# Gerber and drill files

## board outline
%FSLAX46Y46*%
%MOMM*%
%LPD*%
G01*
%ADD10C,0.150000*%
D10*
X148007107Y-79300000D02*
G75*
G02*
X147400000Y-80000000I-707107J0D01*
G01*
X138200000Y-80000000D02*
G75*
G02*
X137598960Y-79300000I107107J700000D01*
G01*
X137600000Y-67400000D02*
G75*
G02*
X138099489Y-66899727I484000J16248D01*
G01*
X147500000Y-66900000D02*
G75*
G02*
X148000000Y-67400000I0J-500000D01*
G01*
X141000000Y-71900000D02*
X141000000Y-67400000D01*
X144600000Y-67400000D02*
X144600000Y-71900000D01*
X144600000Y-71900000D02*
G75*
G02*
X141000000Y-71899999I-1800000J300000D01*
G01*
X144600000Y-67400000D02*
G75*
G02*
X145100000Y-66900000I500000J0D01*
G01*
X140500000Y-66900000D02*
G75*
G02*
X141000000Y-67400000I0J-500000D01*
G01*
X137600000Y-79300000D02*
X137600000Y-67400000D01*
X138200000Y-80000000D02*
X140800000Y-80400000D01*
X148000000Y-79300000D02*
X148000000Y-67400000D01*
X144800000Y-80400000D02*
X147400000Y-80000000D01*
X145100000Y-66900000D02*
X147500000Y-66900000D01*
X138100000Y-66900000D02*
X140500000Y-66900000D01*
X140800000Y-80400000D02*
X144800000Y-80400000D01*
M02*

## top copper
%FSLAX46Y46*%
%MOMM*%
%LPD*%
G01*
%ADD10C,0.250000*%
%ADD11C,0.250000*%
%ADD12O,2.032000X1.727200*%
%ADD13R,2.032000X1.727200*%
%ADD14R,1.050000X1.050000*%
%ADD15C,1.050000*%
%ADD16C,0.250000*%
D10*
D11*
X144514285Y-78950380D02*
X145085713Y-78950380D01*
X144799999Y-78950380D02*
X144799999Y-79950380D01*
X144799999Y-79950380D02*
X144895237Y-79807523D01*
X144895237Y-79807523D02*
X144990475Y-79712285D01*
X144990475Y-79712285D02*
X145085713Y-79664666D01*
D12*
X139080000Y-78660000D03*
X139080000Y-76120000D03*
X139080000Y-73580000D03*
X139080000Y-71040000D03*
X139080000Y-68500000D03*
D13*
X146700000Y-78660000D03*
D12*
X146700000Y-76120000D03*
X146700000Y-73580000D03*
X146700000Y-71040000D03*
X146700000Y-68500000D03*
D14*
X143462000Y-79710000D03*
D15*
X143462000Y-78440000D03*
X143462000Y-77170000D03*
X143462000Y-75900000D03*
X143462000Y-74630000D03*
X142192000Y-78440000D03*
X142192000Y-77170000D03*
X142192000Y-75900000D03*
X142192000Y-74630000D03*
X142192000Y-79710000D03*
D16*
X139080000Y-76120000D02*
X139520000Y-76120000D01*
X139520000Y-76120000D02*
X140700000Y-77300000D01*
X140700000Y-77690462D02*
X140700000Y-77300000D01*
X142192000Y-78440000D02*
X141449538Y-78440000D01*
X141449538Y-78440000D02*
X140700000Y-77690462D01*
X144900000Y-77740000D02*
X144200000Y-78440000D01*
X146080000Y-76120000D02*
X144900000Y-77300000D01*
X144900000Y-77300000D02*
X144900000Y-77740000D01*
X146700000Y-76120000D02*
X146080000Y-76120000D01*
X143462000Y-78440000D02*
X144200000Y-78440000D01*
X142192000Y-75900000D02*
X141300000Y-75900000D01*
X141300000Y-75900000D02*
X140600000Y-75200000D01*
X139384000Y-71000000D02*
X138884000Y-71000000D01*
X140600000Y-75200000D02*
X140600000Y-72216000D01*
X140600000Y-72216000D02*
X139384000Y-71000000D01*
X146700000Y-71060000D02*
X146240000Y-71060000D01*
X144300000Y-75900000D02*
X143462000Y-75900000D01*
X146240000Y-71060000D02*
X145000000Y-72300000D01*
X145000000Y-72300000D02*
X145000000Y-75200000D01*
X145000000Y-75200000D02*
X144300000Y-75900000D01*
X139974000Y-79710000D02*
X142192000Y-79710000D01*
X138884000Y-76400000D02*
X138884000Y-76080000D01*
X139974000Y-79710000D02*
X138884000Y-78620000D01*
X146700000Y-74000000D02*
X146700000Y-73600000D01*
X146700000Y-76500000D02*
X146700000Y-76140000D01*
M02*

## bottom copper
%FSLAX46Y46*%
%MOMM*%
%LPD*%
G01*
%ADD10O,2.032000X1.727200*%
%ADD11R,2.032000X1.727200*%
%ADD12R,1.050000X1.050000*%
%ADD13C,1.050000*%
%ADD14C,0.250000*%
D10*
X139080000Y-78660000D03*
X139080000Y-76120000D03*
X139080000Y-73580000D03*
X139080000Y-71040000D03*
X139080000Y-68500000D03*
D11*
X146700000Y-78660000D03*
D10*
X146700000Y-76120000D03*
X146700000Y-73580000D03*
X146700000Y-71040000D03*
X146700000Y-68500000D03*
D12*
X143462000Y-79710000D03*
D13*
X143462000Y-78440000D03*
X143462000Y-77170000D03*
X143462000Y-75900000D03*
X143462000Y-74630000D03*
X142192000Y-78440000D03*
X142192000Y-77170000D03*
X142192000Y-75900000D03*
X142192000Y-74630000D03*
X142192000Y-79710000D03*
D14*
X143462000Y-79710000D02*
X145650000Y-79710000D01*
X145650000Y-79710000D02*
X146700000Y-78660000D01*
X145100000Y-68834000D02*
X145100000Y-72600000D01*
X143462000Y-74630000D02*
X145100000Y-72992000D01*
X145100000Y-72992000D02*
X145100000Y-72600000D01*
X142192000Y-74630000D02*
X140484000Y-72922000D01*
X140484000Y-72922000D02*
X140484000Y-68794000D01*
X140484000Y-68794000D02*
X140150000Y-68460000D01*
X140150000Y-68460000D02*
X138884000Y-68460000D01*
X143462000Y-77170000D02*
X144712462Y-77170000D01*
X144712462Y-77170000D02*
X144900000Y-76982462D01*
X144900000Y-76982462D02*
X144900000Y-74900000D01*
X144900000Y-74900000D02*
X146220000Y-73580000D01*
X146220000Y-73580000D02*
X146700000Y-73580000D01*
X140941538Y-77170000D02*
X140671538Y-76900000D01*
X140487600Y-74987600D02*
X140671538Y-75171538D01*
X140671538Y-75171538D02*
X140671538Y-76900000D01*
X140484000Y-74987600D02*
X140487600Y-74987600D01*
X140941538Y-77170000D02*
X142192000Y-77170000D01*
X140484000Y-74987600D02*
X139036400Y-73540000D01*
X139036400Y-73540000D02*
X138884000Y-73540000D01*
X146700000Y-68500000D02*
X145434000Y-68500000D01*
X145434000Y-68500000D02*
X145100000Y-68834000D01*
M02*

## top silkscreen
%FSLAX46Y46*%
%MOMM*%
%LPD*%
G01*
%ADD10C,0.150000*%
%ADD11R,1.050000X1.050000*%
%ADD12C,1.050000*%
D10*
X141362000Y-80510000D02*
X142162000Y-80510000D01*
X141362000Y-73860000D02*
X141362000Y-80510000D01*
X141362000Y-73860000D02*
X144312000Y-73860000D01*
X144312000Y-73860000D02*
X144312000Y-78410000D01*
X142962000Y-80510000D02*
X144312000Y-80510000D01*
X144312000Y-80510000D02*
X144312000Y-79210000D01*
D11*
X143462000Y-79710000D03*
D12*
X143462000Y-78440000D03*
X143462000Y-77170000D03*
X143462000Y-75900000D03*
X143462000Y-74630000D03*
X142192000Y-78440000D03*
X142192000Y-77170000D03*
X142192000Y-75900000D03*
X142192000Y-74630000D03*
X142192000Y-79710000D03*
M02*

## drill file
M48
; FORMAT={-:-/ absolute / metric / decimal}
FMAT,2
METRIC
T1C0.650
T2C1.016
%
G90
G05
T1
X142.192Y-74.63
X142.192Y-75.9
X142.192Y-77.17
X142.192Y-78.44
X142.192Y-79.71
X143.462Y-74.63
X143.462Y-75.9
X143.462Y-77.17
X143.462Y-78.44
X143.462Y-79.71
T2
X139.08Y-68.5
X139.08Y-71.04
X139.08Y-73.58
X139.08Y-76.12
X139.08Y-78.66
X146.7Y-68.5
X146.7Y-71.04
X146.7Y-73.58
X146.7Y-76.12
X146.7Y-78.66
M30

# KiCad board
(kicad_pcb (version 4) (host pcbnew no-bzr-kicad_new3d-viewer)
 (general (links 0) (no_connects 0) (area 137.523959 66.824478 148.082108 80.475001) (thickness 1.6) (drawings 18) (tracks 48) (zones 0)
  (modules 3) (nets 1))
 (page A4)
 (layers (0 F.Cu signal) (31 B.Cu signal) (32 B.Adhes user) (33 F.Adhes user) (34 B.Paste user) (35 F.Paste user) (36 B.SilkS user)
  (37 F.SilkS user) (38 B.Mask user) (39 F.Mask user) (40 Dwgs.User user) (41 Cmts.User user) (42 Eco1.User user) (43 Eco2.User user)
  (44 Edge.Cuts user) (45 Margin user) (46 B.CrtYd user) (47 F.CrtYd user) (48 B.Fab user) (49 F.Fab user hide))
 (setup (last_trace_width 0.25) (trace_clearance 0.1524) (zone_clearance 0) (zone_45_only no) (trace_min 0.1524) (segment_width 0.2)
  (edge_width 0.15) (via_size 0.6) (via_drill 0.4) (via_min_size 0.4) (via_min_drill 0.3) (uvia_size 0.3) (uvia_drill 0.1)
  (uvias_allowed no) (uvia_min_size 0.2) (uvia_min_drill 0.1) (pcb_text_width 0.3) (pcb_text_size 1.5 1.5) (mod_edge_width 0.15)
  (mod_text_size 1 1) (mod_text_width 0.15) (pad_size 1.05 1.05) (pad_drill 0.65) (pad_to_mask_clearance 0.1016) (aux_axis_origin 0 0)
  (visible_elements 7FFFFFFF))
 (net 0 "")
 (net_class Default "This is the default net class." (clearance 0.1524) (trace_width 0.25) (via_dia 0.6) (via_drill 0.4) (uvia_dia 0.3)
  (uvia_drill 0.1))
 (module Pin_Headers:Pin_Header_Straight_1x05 (layer B.Cu) (at 139.08 78.66)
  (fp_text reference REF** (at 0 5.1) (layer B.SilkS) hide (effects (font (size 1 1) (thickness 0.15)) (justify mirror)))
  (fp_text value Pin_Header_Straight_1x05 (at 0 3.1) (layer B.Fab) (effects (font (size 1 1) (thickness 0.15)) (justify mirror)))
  (pad 1 thru_hole oval (at 0 0) (size 2.032 1.7272) (drill 1.016) (layers *.Cu *.Mask B.SilkS))
  (pad 2 thru_hole oval (at 0 -2.54) (size 2.032 1.7272) (drill 1.016) (layers *.Cu *.Mask B.SilkS))
  (pad 3 thru_hole oval (at 0 -5.08) (size 2.032 1.7272) (drill 1.016) (layers *.Cu *.Mask B.SilkS))
  (pad 4 thru_hole oval (at 0 -7.62) (size 2.032 1.7272) (drill 1.016) (layers *.Cu *.Mask B.SilkS))
  (pad 5 thru_hole oval (at 0 -10.16) (size 2.032 1.7272) (drill 1.016) (layers *.Cu *.Mask B.SilkS)))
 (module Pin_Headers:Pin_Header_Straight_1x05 (layer B.Cu) (at 146.7 78.66)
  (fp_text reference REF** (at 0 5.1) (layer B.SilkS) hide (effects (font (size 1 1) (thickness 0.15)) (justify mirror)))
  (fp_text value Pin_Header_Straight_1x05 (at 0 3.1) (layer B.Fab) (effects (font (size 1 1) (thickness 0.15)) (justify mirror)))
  (pad 1 thru_hole rect (at 0 0) (size 2.032 1.7272) (drill 1.016) (layers *.Cu *.Mask B.SilkS))
  (pad 2 thru_hole oval (at 0 -2.54) (size 2.032 1.7272) (drill 1.016) (layers *.Cu *.Mask B.SilkS))
  (pad 3 thru_hole oval (at 0 -5.08) (size 2.032 1.7272) (drill 1.016) (layers *.Cu *.Mask B.SilkS))
  (pad 4 thru_hole oval (at 0 -7.62) (size 2.032 1.7272) (drill 1.016) (layers *.Cu *.Mask B.SilkS))
  (pad 5 thru_hole oval (at 0 -10.16) (size 2.032 1.7272) (drill 1.016) (layers *.Cu *.Mask B.SilkS)))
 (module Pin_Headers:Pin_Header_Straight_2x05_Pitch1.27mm (layer F.Cu) (at 143.462 79.71 180)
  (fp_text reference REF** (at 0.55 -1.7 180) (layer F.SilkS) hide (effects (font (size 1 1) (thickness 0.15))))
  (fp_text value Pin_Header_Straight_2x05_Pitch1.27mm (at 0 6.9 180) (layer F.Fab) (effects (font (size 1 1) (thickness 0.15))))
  (fp_line (start 2.1 -0.8) (end 1.3 -0.8) (layer F.SilkS) (width 0.15))
  (fp_line (start 2.1 5.85) (end 2.1 -0.8) (layer F.SilkS) (width 0.15))
  (fp_line (start 2.1 5.85) (end -0.85 5.85) (layer F.SilkS) (width 0.15))
  (fp_line (start -0.85 5.85) (end -0.85 1.3) (layer F.SilkS) (width 0.15))
  (fp_line (start 0.5 -0.8) (end -0.85 -0.8) (layer F.SilkS) (width 0.15))
  (fp_line (start -0.85 -0.8) (end -0.85 0.5) (layer F.SilkS) (width 0.15))
  (pad 1 thru_hole rect (at 0 0 180) (size 1.05 1.05) (drill 0.65) (layers *.Cu *.Mask F.SilkS))
  (pad 3 thru_hole circle (at 0 1.27 180) (size 1.05 1.05) (drill 0.65) (layers *.Cu *.Mask F.SilkS))
  (pad 5 thru_hole circle (at 0 2.54 180) (size 1.05 1.05) (drill 0.65) (layers *.Cu *.Mask F.SilkS))
  (pad 7 thru_hole circle (at 0 3.81 180) (size 1.05 1.05) (drill 0.65) (layers *.Cu *.Mask F.SilkS))
  (pad 9 thru_hole circle (at 0 5.08 180) (size 1.05 1.05) (drill 0.65) (layers *.Cu *.Mask F.SilkS))
  (pad 4 thru_hole circle (at 1.27 1.27 180) (size 1.05 1.05) (drill 0.65) (layers *.Cu *.Mask F.SilkS))
  (pad 6 thru_hole circle (at 1.27 2.54 180) (size 1.05 1.05) (drill 0.65) (layers *.Cu *.Mask F.SilkS))
  (pad 8 thru_hole circle (at 1.27 3.81 180) (size 1.05 1.05) (drill 0.65) (layers *.Cu *.Mask F.SilkS))
  (pad 10 thru_hole circle (at 1.27 5.08 180) (size 1.05 1.05) (drill 0.65) (layers *.Cu *.Mask F.SilkS))
  (pad 2 thru_hole circle (at 1.27 0 180) (size 1.05 1.05) (drill 0.65) (layers *.Cu *.Mask F.SilkS)))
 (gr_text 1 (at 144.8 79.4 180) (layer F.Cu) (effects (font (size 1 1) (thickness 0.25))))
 (gr_arc (start 147.3 79.3) (end 147.4 80) (angle -81.86989765) (layer Edge.Cuts) (width 0.15))
 (gr_arc (start 138.307107 79.3) (end 138.2 80) (angle 81.30064399) (layer Edge.Cuts) (width 0.15))
 (gr_arc (start 138.084 67.383752) (end 137.6 67.4) (angle 93.75557462) (layer Edge.Cuts) (width 0.15))
 (gr_arc (start 147.5 67.4) (end 147.5 66.9) (angle 90) (layer Edge.Cuts) (width 0.15))
 (gr_line (start 141 71.9) (end 141 67.4) (layer Edge.Cuts) (width 0.15))
 (gr_line (start 144.6 67.4) (end 144.6 71.9) (layer Edge.Cuts) (width 0.15))
 (gr_arc (start 142.8 71.6) (end 144.6 71.9) (angle 161.0753866) (layer Edge.Cuts) (width 0.15))
 (gr_arc (start 145.1 67.4) (end 144.6 67.4) (angle 90) (layer Edge.Cuts) (width 0.15))
 (gr_arc (start 140.5 67.4) (end 140.5 66.9) (angle 90) (layer Edge.Cuts) (width 0.15))
 (gr_line (start 137.6 79.3) (end 137.6 67.4) (layer Edge.Cuts) (width 0.15))
 (gr_line (start 138.2 80) (end 140.8 80.4) (layer Edge.Cuts) (width 0.15))
 (gr_line (start 148 79.3) (end 148 67.4) (layer Edge.Cuts) (width 0.15))
 (gr_line (start 144.8 80.4) (end 147.4 80) (layer Edge.Cuts) (width 0.15))
 (gr_line (start 145.1 66.9) (end 147.5 66.9) (layer Edge.Cuts) (width 0.15))
 (gr_line (start 138.1 66.9) (end 140.5 66.9) (layer Edge.Cuts) (width 0.15))
 (gr_line (start 140.8 80.4) (end 144.8 80.4) (layer Edge.Cuts) (width 0.15))
 (segment (start 143.462 79.71) (end 145.65 79.71) (width 0.25) (layer B.Cu) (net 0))
 (segment (start 145.65 79.71) (end 146.7 78.66) (width 0.25) (layer B.Cu) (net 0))
 (segment (start 139.08 76.12) (end 139.52 76.12) (width 0.25) (layer F.Cu) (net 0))
 (segment (start 139.52 76.12) (end 140.7 77.3) (width 0.25) (layer F.Cu) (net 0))
 (segment (start 140.7 77.690462) (end 140.7 77.3) (width 0.25) (layer F.Cu) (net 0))
 (segment (start 142.192 78.44) (end 141.449538 78.44) (width 0.25) (layer F.Cu) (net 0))
 (segment (start 141.449538 78.44) (end 140.7 77.690462) (width 0.25) (layer F.Cu) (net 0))
 (segment (start 144.9 77.74) (end 144.2 78.44) (width 0.25) (layer F.Cu) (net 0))
 (segment (start 146.08 76.12) (end 144.9 77.3) (width 0.25) (layer F.Cu) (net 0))
 (segment (start 144.9 77.3) (end 144.9 77.74) (width 0.25) (layer F.Cu) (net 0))
 (segment (start 146.7 76.12) (end 146.08 76.12) (width 0.25) (layer F.Cu) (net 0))
 (segment (start 143.462 78.44) (end 144.2 78.44) (width 0.25) (layer F.Cu) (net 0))
 (segment (start 142.192 75.9) (end 141.3 75.9) (width 0.25) (layer F.Cu) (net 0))
 (segment (start 141.3 75.9) (end 140.6 75.2) (width 0.25) (layer F.Cu) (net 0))
 (segment (start 139.384 71) (end 138.884 71) (width 0.25) (layer F.Cu) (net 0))
 (segment (start 140.6 75.2) (end 140.6 72.216) (width 0.25) (layer F.Cu) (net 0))
 (segment (start 140.6 72.216) (end 139.384 71) (width 0.25) (layer F.Cu) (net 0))
 (segment (start 146.7 71.06) (end 146.24 71.06) (width 0.25) (layer F.Cu) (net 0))
 (segment (start 144.3 75.9) (end 143.462 75.9) (width 0.25) (layer F.Cu) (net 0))
 (segment (start 146.24 71.06) (end 145 72.3) (width 0.25) (layer F.Cu) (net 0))
 (segment (start 145 72.3) (end 145 75.2) (width 0.25) (layer F.Cu) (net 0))
 (segment (start 145 75.2) (end 144.3 75.9) (width 0.25) (layer F.Cu) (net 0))
 (segment (start 145.1 68.834) (end 145.1 72.6) (width 0.25) (layer B.Cu) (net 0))
 (segment (start 143.462 74.63) (end 145.1 72.992) (width 0.25) (layer B.Cu) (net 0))
 (segment (start 145.1 72.992) (end 145.1 72.6) (width 0.25) (layer B.Cu) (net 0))
 (segment (start 142.192 74.63) (end 140.484 72.922) (width 0.25) (layer B.Cu) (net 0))
 (segment (start 140.484 72.922) (end 140.484 68.794) (width 0.25) (layer B.Cu) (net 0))
 (segment (start 140.484 68.794) (end 140.15 68.46) (width 0.25) (layer B.Cu) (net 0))
 (segment (start 140.15 68.46) (end 138.884 68.46) (width 0.25) (layer B.Cu) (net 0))
 (segment (start 143.462 77.17) (end 144.712462 77.17) (width 0.25) (layer B.Cu) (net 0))
 (segment (start 144.712462 77.17) (end 144.9 76.982462) (width 0.25) (layer B.Cu) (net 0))
 (segment (start 144.9 76.982462) (end 144.9 74.9) (width 0.25) (layer B.Cu) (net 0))
 (segment (start 144.9 74.9) (end 146.22 73.58) (width 0.25) (layer B.Cu) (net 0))
 (segment (start 146.22 73.58) (end 146.7 73.58) (width 0.25) (layer B.Cu) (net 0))
 (segment (start 140.941538 77.17) (end 140.671538 76.9) (width 0.25) (layer B.Cu) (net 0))
 (segment (start 140.4876 74.9876) (end 140.671538 75.171538) (width 0.25) (layer B.Cu) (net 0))
 (segment (start 140.671538 75.171538) (end 140.671538 76.9) (width 0.25) (layer B.Cu) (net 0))
 (segment (start 140.484 74.9876) (end 140.4876 74.9876) (width 0.25) (layer B.Cu) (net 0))
 (segment (start 140.941538 77.17) (end 142.192 77.17) (width 0.25) (layer B.Cu) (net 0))
 (segment (start 139.974 79.71) (end 142.192 79.71) (width 0.25) (layer F.Cu) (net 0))
 (segment (start 138.884 76.4) (end 138.884 76.08) (width 0.25) (layer F.Cu) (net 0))
 (segment (start 139.974 79.71) (end 138.884 78.62) (width 0.25) (layer F.Cu) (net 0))
 (segment (start 140.484 74.9876) (end 139.0364 73.54) (width 0.25) (layer B.Cu) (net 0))
 (segment (start 139.0364 73.54) (end 138.884 73.54) (width 0.25) (layer B.Cu) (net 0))
 (segment (start 146.7 68.5) (end 145.434 68.5) (width 0.25) (layer B.Cu) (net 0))
 (segment (start 145.434 68.5) (end 145.1 68.834) (width 0.25) (layer B.Cu) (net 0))
 (segment (start 146.7 74) (end 146.7 73.6) (width 0.25) (layer F.Cu) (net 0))
 (segment (start 146.7 76.5) (end 146.7 76.14) (width 0.25) (layer F.Cu) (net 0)))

